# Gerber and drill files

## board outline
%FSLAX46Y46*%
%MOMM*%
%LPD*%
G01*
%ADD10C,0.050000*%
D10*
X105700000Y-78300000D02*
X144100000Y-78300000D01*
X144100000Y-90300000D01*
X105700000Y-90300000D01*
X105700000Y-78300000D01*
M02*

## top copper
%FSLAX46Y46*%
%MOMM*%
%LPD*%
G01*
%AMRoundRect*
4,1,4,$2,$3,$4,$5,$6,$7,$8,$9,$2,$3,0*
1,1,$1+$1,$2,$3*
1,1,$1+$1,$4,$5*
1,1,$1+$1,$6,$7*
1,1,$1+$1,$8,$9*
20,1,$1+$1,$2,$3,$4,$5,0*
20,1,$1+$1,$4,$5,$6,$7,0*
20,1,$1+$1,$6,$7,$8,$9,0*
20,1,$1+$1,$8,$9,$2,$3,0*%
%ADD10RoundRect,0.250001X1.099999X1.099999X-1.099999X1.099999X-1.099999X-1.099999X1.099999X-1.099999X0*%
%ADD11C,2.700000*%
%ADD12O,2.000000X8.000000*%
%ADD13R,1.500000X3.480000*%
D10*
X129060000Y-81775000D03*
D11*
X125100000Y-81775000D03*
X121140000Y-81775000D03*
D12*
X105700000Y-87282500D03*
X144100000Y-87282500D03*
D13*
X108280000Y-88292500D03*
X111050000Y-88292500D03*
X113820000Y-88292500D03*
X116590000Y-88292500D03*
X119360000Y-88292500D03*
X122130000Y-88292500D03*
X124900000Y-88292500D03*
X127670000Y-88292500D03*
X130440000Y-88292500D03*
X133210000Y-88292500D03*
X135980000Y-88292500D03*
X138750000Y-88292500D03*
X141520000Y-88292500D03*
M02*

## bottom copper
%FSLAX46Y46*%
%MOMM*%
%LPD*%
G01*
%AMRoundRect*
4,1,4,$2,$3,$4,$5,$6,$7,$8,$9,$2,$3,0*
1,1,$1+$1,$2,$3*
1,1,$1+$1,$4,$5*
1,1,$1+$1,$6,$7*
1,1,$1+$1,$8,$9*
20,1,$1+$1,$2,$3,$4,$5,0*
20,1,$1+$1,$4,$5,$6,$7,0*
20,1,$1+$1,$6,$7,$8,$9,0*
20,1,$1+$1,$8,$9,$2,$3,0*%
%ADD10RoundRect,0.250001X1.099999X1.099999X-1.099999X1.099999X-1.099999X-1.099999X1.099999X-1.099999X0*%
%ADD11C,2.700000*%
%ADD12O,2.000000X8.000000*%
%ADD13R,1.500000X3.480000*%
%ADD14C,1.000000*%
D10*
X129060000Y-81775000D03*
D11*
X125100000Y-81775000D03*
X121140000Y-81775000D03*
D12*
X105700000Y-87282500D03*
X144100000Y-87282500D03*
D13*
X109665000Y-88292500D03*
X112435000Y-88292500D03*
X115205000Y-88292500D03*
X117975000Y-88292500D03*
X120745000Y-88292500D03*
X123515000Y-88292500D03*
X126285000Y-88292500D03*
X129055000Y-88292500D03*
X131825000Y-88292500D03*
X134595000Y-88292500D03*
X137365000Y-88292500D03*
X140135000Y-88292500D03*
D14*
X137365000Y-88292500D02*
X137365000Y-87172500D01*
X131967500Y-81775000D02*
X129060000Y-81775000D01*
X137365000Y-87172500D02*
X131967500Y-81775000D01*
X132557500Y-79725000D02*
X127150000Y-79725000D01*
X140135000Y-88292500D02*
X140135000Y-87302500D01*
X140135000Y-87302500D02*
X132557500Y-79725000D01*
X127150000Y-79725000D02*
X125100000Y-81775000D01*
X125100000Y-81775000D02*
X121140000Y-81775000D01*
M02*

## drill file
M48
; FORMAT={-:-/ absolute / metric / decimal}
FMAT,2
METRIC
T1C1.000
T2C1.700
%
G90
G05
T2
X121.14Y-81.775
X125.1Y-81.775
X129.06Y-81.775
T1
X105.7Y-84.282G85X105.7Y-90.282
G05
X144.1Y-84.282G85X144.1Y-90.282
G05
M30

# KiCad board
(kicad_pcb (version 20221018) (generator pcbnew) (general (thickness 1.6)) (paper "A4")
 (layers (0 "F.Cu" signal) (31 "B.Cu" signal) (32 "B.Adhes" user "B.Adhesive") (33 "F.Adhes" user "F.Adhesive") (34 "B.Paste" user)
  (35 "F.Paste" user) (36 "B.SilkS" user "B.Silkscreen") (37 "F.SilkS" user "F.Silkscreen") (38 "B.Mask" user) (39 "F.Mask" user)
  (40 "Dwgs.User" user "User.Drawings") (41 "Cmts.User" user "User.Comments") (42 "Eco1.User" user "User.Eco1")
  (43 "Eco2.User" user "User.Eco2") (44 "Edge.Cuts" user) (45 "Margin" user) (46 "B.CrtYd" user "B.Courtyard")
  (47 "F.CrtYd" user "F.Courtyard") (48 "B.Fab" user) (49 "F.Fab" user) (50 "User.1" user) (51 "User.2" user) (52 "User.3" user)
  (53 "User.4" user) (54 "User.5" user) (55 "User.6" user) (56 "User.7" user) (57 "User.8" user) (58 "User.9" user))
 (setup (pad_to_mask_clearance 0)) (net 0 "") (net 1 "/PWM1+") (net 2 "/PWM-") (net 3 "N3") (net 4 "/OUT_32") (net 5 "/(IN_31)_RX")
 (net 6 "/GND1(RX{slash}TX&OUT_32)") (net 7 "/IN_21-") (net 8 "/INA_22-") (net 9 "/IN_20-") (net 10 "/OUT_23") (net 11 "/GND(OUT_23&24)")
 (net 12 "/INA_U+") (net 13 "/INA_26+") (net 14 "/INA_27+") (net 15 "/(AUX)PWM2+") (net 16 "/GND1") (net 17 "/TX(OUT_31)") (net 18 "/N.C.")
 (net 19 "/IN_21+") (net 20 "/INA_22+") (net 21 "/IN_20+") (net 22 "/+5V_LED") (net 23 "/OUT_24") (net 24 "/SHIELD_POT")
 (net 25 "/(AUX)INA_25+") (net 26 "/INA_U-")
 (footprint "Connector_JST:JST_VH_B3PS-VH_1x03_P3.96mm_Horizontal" (layer "F.Cu") (at 129.06 81.775 180)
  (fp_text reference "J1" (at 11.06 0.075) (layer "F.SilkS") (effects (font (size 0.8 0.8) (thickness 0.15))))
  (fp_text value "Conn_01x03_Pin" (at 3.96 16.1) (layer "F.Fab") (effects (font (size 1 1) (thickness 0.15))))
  (pad "1" thru_hole roundrect (at 0 0 180) (size 2.7 2.7) (drill 1.7) (layers "*.Cu" "*.Mask") (roundrect_rratio 0.092593) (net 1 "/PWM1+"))
  (pad "2" thru_hole circle (at 3.96 0 180) (size 2.7 2.7) (drill 1.7) (layers "*.Cu" "*.Mask") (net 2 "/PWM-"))
  (pad "3" thru_hole circle (at 7.92 0 180) (size 2.7 2.7) (drill 1.7) (layers "*.Cu" "*.Mask") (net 2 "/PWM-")))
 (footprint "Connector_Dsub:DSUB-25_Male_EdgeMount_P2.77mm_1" (layer "F.Cu") (at 124.9 88.2925)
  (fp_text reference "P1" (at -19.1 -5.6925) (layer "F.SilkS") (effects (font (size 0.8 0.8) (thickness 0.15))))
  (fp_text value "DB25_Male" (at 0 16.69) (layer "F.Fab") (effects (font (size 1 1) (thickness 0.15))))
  (pad "0" thru_hole oval (at -19.2 -1.01) (size 2 8) (drill oval 1 7) (layers "*.Cu" "*.Mask") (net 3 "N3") (thermal_bridge_angle 45))
  (pad "0" thru_hole oval (at 19.2 -1.01) (size 2 8) (drill oval 1 7) (layers "*.Cu" "*.Mask") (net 3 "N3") (thermal_bridge_angle 45))
  (pad "1" smd rect (at -16.62 0) (size 1.5 3.48) (layers "F.Cu" "F.Paste" "F.Mask") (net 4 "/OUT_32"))
  (pad "2" smd rect (at -13.85 0) (size 1.5 3.48) (layers "F.Cu" "F.Paste" "F.Mask") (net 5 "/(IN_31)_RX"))
  (pad "3" smd rect (at -11.08 0) (size 1.5 3.48) (layers "F.Cu" "F.Paste" "F.Mask") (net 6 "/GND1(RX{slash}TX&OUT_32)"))
  (pad "4" smd rect (at -8.31 0) (size 1.5 3.48) (layers "F.Cu" "F.Paste" "F.Mask") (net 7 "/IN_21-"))
  (pad "5" smd rect (at -5.54 0) (size 1.5 3.48) (layers "F.Cu" "F.Paste" "F.Mask") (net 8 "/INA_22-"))
  (pad "6" smd rect (at -2.77 0) (size 1.5 3.48) (layers "F.Cu" "F.Paste" "F.Mask") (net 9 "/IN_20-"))
  (pad "7" smd rect (at 0 0) (size 1.5 3.48) (layers "F.Cu" "F.Paste" "F.Mask") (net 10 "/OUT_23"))
  (pad "8" smd rect (at 2.77 0) (size 1.5 3.48) (layers "F.Cu" "F.Paste" "F.Mask") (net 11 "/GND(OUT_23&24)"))
  (pad "9" smd rect (at 5.54 0) (size 1.5 3.48) (layers "F.Cu" "F.Paste" "F.Mask") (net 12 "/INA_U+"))
  (pad "10" smd rect (at 8.31 0) (size 1.5 3.48) (layers "F.Cu" "F.Paste" "F.Mask") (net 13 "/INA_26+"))
  (pad "11" smd rect (at 11.08 0) (size 1.5 3.48) (layers "F.Cu" "F.Paste" "F.Mask") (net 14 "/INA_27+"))
  (pad "12" smd rect (at 13.85 0) (size 1.5 3.48) (layers "F.Cu" "F.Paste" "F.Mask") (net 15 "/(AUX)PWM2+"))
  (pad "13" smd rect (at 16.62 0) (size 1.5 3.48) (layers "F.Cu" "F.Paste" "F.Mask") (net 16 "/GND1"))
  (pad "14" smd rect (at -15.235 0) (size 1.5 3.48) (layers "B.Cu" "B.Paste" "B.Mask") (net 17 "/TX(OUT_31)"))
  (pad "15" smd rect (at -12.465 0) (size 1.5 3.48) (layers "B.Cu" "B.Paste" "B.Mask") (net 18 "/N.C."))
  (pad "16" smd rect (at -9.695 0) (size 1.5 3.48) (layers "B.Cu" "B.Paste" "B.Mask") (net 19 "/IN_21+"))
  (pad "17" smd rect (at -6.925 0) (size 1.5 3.48) (layers "B.Cu" "B.Paste" "B.Mask") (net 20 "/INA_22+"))
  (pad "18" smd rect (at -4.155 0) (size 1.5 3.48) (layers "B.Cu" "B.Paste" "B.Mask") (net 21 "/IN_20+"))
  (pad "19" smd rect (at -1.385 0) (size 1.5 3.48) (layers "B.Cu" "B.Paste" "B.Mask") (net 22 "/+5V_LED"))
  (pad "20" smd rect (at 1.385 0) (size 1.5 3.48) (layers "B.Cu" "B.Paste" "B.Mask") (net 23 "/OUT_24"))
  (pad "21" smd rect (at 4.155 0) (size 1.5 3.48) (layers "B.Cu" "B.Paste" "B.Mask") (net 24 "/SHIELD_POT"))
  (pad "22" smd rect (at 6.925 0) (size 1.5 3.48) (layers "B.Cu" "B.Paste" "B.Mask") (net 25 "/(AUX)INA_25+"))
  (pad "23" smd rect (at 9.695 0) (size 1.5 3.48) (layers "B.Cu" "B.Paste" "B.Mask") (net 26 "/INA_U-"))
  (pad "24" smd rect (at 12.465 0) (size 1.5 3.48) (layers "B.Cu" "B.Paste" "B.Mask") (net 1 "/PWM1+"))
  (pad "25" smd rect (at 15.235 0) (size 1.5 3.48) (layers "B.Cu" "B.Paste" "B.Mask") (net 2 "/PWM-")))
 (gr_rect (start 105.7 78.3) (end 144.1 90.3) (stroke (width 0.05) (type default)) (fill none) (layer "Edge.Cuts"))
 (segment (start 137.365 88.2925) (end 137.365 87.1725) (width 1) (layer "B.Cu") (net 1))
 (segment (start 131.9675 81.775) (end 129.06 81.775) (width 1) (layer "B.Cu") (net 1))
 (segment (start 137.365 87.1725) (end 131.9675 81.775) (width 1) (layer "B.Cu") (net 1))
 (segment (start 132.5575 79.725) (end 127.15 79.725) (width 1) (layer "B.Cu") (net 2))
 (segment (start 140.135 88.2925) (end 140.135 87.3025) (width 1) (layer "B.Cu") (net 2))
 (segment (start 140.135 87.3025) (end 132.5575 79.725) (width 1) (layer "B.Cu") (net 2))
 (segment (start 127.15 79.725) (end 125.1 81.775) (width 1) (layer "B.Cu") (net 2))
 (segment (start 125.1 81.775) (end 121.14 81.775) (width 1) (layer "B.Cu") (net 2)))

